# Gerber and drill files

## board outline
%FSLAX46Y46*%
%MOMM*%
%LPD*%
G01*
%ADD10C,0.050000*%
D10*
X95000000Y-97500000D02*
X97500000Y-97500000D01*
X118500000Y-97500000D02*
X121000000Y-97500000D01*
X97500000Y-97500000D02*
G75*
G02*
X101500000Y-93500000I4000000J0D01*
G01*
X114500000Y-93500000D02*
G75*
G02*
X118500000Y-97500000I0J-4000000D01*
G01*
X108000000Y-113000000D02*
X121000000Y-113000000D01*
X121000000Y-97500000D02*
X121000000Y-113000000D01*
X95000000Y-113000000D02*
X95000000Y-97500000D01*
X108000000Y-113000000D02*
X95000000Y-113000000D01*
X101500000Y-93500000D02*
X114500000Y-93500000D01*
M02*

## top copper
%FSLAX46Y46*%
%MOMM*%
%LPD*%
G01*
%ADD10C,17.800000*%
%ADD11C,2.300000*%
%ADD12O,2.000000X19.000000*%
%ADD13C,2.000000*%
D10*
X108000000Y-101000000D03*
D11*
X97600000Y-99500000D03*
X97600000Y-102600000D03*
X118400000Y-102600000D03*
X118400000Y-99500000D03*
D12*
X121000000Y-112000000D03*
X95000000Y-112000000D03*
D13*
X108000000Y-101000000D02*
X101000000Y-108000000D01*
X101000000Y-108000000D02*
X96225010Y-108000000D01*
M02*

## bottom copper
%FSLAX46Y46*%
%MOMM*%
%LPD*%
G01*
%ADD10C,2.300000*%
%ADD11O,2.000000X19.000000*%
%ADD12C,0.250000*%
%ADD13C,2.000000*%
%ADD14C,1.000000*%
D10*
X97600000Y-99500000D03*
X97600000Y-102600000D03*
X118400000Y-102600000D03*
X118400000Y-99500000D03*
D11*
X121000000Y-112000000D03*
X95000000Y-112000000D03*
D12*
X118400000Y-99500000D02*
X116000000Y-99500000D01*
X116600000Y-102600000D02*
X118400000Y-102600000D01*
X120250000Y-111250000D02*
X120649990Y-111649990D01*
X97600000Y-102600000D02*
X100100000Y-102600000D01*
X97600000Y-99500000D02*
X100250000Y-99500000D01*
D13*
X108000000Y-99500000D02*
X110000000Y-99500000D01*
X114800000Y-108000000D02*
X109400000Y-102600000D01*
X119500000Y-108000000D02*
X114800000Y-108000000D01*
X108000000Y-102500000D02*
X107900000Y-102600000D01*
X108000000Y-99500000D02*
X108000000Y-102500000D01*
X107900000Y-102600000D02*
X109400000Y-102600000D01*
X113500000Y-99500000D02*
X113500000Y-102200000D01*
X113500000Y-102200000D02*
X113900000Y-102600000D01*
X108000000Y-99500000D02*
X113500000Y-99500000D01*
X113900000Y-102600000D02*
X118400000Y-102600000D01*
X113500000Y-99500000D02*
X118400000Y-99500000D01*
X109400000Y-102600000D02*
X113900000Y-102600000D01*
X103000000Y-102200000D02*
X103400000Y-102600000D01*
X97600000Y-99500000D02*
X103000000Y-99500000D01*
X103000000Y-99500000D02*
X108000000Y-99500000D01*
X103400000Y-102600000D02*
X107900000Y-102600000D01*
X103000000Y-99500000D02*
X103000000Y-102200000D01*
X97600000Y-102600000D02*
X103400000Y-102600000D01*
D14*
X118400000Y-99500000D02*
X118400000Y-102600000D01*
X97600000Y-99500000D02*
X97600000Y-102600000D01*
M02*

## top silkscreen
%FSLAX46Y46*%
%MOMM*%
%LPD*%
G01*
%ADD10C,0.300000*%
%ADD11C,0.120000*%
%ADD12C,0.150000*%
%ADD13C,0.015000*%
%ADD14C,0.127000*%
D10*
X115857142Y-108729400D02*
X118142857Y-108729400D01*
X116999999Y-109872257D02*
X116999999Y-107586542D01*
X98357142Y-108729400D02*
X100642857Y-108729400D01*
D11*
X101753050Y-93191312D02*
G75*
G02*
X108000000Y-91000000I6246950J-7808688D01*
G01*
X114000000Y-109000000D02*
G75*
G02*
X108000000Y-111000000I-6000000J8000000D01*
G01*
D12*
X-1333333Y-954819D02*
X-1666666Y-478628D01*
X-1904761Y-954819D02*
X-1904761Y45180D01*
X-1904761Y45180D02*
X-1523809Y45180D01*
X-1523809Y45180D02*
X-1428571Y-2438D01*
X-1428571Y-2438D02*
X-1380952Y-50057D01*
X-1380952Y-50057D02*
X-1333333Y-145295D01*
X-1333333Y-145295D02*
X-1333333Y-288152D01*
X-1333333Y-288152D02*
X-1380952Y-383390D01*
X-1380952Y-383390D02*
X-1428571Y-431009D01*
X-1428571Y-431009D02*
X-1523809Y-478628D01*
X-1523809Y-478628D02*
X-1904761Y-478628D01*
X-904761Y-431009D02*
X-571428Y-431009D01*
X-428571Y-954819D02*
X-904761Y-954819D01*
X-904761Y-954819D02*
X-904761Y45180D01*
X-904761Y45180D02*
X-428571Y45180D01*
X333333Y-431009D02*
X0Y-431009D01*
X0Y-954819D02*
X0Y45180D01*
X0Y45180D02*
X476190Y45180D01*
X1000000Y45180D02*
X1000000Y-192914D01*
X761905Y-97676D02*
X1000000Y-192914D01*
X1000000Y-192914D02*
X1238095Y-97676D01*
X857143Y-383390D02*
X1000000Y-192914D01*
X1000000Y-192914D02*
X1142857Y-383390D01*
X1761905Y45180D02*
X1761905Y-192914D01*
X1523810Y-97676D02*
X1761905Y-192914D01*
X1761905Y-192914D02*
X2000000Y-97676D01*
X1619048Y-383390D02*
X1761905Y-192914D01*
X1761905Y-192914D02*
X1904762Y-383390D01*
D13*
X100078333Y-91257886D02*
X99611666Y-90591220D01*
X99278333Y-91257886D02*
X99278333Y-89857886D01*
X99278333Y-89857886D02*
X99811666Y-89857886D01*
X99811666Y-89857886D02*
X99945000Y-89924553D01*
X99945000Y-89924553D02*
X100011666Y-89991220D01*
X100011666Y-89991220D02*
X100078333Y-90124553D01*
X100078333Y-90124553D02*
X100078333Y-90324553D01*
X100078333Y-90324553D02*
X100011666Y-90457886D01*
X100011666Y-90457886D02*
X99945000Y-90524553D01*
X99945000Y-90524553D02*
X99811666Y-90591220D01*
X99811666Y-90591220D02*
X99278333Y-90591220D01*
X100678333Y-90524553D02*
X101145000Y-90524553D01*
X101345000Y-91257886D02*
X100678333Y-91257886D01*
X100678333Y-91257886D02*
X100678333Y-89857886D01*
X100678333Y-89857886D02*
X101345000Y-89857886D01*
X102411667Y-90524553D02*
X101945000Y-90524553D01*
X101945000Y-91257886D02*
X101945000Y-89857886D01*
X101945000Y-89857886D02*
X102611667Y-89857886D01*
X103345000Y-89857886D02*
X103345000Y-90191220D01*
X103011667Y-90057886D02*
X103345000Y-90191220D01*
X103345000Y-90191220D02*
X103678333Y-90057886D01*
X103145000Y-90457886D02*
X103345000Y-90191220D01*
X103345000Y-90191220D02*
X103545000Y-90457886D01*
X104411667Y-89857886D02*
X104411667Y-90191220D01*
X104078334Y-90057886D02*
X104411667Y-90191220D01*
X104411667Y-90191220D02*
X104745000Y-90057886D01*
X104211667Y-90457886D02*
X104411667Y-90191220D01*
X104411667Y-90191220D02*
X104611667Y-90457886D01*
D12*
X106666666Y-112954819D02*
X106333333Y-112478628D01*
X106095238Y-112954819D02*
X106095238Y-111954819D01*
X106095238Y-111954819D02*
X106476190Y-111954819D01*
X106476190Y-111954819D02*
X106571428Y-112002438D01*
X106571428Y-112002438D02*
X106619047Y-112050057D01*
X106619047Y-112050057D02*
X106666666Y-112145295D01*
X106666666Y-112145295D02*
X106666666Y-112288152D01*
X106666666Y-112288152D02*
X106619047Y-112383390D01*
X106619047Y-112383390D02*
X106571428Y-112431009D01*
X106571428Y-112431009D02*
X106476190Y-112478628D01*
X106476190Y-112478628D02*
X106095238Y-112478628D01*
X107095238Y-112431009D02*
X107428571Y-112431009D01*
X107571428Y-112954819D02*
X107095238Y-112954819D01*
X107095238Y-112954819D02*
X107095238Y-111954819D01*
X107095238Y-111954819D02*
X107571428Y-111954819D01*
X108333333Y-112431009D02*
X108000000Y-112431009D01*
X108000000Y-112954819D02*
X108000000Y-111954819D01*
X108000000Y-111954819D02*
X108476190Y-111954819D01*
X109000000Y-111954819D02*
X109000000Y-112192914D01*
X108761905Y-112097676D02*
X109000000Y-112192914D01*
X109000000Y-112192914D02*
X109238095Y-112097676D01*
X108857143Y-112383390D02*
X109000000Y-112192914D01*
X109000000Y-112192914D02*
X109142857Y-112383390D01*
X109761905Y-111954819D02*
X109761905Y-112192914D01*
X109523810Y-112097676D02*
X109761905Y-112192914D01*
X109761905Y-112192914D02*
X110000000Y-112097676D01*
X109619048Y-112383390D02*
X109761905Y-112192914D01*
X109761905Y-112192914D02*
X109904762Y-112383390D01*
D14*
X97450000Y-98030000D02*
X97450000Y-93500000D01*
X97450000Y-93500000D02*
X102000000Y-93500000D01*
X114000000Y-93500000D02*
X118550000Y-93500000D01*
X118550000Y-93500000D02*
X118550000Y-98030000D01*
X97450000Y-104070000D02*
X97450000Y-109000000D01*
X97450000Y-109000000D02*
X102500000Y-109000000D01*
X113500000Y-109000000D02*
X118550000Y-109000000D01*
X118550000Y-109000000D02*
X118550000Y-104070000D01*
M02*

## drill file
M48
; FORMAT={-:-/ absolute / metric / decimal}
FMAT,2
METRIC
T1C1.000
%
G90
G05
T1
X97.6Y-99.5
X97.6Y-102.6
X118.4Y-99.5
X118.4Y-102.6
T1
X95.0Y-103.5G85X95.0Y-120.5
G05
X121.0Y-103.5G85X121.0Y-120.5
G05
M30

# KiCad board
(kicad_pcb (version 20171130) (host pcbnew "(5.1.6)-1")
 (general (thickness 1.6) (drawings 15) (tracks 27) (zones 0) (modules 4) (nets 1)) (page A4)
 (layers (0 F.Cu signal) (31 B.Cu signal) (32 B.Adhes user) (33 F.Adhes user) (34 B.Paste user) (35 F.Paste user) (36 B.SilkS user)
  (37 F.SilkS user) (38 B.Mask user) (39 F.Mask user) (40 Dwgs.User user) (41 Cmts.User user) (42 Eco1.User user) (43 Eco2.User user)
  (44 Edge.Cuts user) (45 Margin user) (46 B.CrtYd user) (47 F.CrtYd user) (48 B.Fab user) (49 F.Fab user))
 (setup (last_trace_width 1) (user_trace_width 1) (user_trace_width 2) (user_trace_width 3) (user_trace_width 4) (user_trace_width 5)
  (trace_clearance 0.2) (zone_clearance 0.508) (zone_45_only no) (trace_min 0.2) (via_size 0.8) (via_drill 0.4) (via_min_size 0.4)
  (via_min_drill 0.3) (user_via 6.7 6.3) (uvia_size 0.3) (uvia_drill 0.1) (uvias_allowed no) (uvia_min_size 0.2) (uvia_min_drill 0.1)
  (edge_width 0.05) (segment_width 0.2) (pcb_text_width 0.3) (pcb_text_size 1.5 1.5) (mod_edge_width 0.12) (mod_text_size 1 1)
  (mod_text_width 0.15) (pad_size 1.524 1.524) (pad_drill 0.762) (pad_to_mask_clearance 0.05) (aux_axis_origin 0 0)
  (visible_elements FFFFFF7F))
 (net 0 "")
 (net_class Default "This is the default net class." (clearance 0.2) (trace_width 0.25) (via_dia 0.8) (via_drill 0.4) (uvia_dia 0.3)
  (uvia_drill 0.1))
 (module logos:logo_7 (layer F.Cu) (at 103.5 101.5)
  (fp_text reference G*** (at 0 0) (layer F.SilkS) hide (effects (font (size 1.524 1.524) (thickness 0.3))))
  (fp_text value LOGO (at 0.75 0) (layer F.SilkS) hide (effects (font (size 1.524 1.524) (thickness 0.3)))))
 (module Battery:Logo (layer F.Cu) (at 0 0)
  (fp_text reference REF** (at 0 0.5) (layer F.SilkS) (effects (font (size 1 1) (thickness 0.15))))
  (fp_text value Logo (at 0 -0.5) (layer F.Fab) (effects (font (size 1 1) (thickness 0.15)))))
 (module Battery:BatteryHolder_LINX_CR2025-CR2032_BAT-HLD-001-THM (layer F.Cu) (at 108 101)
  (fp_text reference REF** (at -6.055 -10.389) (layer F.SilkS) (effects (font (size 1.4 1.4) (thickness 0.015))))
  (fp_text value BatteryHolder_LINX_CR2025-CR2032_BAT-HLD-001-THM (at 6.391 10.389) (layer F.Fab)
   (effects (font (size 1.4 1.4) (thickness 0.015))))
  (fp_line (start -10.55 -2.97) (end -10.55 -7.5) (layer F.SilkS) (width 0.127))
  (fp_line (start -10.55 -7.5) (end -6 -7.5) (layer F.SilkS) (width 0.127))
  (fp_line (start 6 -7.5) (end 10.55 -7.5) (layer F.SilkS) (width 0.127))
  (fp_line (start 10.55 -7.5) (end 10.55 -2.97) (layer F.SilkS) (width 0.127))
  (fp_line (start -10.55 3.07) (end -10.55 8) (layer F.SilkS) (width 0.127))
  (fp_line (start -10.55 8) (end -5.5 8) (layer F.SilkS) (width 0.127))
  (fp_line (start 5.5 8) (end 10.55 8) (layer F.SilkS) (width 0.127))
  (fp_line (start 10.55 8) (end 10.55 3.07) (layer F.SilkS) (width 0.127))
  (pad N smd circle (at 0 0) (size 17.8 17.8) (layers F.Cu F.Mask))
  (pad P1 thru_hole circle (at -10.4 -1.5) (size 2.3 2.3) (drill 1) (layers *.Cu *.Mask))
  (pad P2 thru_hole circle (at -10.4 1.6) (size 2.3 2.3) (drill 1) (layers *.Cu *.Mask))
  (pad P3 thru_hole circle (at 10.4 1.6) (size 2.3 2.3) (drill 1) (layers *.Cu *.Mask))
  (pad P4 thru_hole circle (at 10.4 -1.5) (size 2.3 2.3) (drill 1) (layers *.Cu *.Mask)))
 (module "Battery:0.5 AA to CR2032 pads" (layer F.Cu) (at 108 112)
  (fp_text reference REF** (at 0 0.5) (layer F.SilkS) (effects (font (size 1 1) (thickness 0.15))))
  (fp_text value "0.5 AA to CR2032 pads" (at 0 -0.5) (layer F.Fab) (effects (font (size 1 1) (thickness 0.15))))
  (pad 2 thru_hole oval (at 13 0) (size 2 19) (drill oval 1 18) (layers *.Cu *.Mask))
  (pad 1 thru_hole oval (at -13 0) (size 2 19) (drill oval 1 18) (layers *.Cu *.Mask)))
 (gr_line (start 95 97.5) (end 97.5 97.5) (layer Edge.Cuts) (width 0.05))
 (gr_line (start 118.5 97.5) (end 121 97.5) (layer Edge.Cuts) (width 0.05))
 (gr_arc (start 101.5 97.5) (end 101.5 93.5) (angle -90) (layer Edge.Cuts) (width 0.05))
 (gr_arc (start 114.5 97.5) (end 118.5 97.5) (angle -90) (layer Edge.Cuts) (width 0.05))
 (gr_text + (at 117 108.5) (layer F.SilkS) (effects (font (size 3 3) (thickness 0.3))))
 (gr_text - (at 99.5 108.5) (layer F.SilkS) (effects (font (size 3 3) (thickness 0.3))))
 (gr_line (start 108 113) (end 121 113) (layer Edge.Cuts) (width 0.05))
 (gr_line (start 121 97.5) (end 121 113) (layer Edge.Cuts) (width 0.05))
 (gr_line (start 95 113) (end 95 97.5) (layer Edge.Cuts) (width 0.05))
 (gr_line (start 108 113) (end 95 113) (layer Edge.Cuts) (width 0.05))
 (gr_line (start 101.5 93.5) (end 114.5 93.5) (layer Edge.Cuts) (width 0.05))
 (gr_arc (start 108 101) (end 108 91) (angle -38.65980825) (layer F.SilkS) (width 0.12))
 (gr_arc (start 108 101) (end 108 111) (angle -36.86989765) (layer F.SilkS) (width 0.12))
 (segment (start 118.4 99.5) (end 116 99.5) (width 0.25) (layer B.Cu) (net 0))
 (segment (start 116.6 102.6) (end 118.4 102.6) (width 0.25) (layer B.Cu) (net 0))
 (segment (start 120.25 111.25) (end 120.64999 111.64999) (width 0.25) (layer B.Cu) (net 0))
 (segment (start 97.6 102.6) (end 100.1 102.6) (width 0.25) (layer B.Cu) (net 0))
 (segment (start 97.6 99.5) (end 100.25 99.5) (width 0.25) (layer B.Cu) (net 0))
 (segment (start 108 101) (end 101 108) (width 2) (layer F.Cu) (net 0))
 (segment (start 101 108) (end 96.22501 108) (width 2) (layer F.Cu) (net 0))
 (segment (start 108 99.5) (end 110 99.5) (width 2) (layer B.Cu) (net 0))
 (segment (start 114.8 108) (end 109.4 102.6) (width 2) (layer B.Cu) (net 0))
 (segment (start 119.5 108) (end 114.8 108) (width 2) (layer B.Cu) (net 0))
 (segment (start 108 102.5) (end 107.9 102.6) (width 2) (layer B.Cu) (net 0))
 (segment (start 108 99.5) (end 108 102.5) (width 2) (layer B.Cu) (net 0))
 (segment (start 107.9 102.6) (end 109.4 102.6) (width 2) (layer B.Cu) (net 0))
 (segment (start 113.5 99.5) (end 113.5 102.2) (width 2) (layer B.Cu) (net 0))
 (segment (start 113.5 102.2) (end 113.9 102.6) (width 2) (layer B.Cu) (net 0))
 (segment (start 108 99.5) (end 113.5 99.5) (width 2) (layer B.Cu) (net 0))
 (segment (start 113.9 102.6) (end 118.4 102.6) (width 2) (layer B.Cu) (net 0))
 (segment (start 113.5 99.5) (end 118.4 99.5) (width 2) (layer B.Cu) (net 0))
 (segment (start 109.4 102.6) (end 113.9 102.6) (width 2) (layer B.Cu) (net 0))
 (segment (start 103 102.2) (end 103.4 102.6) (width 2) (layer B.Cu) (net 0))
 (segment (start 97.6 99.5) (end 103 99.5) (width 2) (layer B.Cu) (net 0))
 (segment (start 103 99.5) (end 108 99.5) (width 2) (layer B.Cu) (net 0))
 (segment (start 103.4 102.6) (end 107.9 102.6) (width 2) (layer B.Cu) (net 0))
 (segment (start 103 99.5) (end 103 102.2) (width 2) (layer B.Cu) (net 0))
 (segment (start 97.6 102.6) (end 103.4 102.6) (width 2) (layer B.Cu) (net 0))
 (segment (start 118.4 99.5) (end 118.4 102.6) (width 1) (layer B.Cu) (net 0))
 (segment (start 97.6 99.5) (end 97.6 102.6) (width 1) (layer B.Cu) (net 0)))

